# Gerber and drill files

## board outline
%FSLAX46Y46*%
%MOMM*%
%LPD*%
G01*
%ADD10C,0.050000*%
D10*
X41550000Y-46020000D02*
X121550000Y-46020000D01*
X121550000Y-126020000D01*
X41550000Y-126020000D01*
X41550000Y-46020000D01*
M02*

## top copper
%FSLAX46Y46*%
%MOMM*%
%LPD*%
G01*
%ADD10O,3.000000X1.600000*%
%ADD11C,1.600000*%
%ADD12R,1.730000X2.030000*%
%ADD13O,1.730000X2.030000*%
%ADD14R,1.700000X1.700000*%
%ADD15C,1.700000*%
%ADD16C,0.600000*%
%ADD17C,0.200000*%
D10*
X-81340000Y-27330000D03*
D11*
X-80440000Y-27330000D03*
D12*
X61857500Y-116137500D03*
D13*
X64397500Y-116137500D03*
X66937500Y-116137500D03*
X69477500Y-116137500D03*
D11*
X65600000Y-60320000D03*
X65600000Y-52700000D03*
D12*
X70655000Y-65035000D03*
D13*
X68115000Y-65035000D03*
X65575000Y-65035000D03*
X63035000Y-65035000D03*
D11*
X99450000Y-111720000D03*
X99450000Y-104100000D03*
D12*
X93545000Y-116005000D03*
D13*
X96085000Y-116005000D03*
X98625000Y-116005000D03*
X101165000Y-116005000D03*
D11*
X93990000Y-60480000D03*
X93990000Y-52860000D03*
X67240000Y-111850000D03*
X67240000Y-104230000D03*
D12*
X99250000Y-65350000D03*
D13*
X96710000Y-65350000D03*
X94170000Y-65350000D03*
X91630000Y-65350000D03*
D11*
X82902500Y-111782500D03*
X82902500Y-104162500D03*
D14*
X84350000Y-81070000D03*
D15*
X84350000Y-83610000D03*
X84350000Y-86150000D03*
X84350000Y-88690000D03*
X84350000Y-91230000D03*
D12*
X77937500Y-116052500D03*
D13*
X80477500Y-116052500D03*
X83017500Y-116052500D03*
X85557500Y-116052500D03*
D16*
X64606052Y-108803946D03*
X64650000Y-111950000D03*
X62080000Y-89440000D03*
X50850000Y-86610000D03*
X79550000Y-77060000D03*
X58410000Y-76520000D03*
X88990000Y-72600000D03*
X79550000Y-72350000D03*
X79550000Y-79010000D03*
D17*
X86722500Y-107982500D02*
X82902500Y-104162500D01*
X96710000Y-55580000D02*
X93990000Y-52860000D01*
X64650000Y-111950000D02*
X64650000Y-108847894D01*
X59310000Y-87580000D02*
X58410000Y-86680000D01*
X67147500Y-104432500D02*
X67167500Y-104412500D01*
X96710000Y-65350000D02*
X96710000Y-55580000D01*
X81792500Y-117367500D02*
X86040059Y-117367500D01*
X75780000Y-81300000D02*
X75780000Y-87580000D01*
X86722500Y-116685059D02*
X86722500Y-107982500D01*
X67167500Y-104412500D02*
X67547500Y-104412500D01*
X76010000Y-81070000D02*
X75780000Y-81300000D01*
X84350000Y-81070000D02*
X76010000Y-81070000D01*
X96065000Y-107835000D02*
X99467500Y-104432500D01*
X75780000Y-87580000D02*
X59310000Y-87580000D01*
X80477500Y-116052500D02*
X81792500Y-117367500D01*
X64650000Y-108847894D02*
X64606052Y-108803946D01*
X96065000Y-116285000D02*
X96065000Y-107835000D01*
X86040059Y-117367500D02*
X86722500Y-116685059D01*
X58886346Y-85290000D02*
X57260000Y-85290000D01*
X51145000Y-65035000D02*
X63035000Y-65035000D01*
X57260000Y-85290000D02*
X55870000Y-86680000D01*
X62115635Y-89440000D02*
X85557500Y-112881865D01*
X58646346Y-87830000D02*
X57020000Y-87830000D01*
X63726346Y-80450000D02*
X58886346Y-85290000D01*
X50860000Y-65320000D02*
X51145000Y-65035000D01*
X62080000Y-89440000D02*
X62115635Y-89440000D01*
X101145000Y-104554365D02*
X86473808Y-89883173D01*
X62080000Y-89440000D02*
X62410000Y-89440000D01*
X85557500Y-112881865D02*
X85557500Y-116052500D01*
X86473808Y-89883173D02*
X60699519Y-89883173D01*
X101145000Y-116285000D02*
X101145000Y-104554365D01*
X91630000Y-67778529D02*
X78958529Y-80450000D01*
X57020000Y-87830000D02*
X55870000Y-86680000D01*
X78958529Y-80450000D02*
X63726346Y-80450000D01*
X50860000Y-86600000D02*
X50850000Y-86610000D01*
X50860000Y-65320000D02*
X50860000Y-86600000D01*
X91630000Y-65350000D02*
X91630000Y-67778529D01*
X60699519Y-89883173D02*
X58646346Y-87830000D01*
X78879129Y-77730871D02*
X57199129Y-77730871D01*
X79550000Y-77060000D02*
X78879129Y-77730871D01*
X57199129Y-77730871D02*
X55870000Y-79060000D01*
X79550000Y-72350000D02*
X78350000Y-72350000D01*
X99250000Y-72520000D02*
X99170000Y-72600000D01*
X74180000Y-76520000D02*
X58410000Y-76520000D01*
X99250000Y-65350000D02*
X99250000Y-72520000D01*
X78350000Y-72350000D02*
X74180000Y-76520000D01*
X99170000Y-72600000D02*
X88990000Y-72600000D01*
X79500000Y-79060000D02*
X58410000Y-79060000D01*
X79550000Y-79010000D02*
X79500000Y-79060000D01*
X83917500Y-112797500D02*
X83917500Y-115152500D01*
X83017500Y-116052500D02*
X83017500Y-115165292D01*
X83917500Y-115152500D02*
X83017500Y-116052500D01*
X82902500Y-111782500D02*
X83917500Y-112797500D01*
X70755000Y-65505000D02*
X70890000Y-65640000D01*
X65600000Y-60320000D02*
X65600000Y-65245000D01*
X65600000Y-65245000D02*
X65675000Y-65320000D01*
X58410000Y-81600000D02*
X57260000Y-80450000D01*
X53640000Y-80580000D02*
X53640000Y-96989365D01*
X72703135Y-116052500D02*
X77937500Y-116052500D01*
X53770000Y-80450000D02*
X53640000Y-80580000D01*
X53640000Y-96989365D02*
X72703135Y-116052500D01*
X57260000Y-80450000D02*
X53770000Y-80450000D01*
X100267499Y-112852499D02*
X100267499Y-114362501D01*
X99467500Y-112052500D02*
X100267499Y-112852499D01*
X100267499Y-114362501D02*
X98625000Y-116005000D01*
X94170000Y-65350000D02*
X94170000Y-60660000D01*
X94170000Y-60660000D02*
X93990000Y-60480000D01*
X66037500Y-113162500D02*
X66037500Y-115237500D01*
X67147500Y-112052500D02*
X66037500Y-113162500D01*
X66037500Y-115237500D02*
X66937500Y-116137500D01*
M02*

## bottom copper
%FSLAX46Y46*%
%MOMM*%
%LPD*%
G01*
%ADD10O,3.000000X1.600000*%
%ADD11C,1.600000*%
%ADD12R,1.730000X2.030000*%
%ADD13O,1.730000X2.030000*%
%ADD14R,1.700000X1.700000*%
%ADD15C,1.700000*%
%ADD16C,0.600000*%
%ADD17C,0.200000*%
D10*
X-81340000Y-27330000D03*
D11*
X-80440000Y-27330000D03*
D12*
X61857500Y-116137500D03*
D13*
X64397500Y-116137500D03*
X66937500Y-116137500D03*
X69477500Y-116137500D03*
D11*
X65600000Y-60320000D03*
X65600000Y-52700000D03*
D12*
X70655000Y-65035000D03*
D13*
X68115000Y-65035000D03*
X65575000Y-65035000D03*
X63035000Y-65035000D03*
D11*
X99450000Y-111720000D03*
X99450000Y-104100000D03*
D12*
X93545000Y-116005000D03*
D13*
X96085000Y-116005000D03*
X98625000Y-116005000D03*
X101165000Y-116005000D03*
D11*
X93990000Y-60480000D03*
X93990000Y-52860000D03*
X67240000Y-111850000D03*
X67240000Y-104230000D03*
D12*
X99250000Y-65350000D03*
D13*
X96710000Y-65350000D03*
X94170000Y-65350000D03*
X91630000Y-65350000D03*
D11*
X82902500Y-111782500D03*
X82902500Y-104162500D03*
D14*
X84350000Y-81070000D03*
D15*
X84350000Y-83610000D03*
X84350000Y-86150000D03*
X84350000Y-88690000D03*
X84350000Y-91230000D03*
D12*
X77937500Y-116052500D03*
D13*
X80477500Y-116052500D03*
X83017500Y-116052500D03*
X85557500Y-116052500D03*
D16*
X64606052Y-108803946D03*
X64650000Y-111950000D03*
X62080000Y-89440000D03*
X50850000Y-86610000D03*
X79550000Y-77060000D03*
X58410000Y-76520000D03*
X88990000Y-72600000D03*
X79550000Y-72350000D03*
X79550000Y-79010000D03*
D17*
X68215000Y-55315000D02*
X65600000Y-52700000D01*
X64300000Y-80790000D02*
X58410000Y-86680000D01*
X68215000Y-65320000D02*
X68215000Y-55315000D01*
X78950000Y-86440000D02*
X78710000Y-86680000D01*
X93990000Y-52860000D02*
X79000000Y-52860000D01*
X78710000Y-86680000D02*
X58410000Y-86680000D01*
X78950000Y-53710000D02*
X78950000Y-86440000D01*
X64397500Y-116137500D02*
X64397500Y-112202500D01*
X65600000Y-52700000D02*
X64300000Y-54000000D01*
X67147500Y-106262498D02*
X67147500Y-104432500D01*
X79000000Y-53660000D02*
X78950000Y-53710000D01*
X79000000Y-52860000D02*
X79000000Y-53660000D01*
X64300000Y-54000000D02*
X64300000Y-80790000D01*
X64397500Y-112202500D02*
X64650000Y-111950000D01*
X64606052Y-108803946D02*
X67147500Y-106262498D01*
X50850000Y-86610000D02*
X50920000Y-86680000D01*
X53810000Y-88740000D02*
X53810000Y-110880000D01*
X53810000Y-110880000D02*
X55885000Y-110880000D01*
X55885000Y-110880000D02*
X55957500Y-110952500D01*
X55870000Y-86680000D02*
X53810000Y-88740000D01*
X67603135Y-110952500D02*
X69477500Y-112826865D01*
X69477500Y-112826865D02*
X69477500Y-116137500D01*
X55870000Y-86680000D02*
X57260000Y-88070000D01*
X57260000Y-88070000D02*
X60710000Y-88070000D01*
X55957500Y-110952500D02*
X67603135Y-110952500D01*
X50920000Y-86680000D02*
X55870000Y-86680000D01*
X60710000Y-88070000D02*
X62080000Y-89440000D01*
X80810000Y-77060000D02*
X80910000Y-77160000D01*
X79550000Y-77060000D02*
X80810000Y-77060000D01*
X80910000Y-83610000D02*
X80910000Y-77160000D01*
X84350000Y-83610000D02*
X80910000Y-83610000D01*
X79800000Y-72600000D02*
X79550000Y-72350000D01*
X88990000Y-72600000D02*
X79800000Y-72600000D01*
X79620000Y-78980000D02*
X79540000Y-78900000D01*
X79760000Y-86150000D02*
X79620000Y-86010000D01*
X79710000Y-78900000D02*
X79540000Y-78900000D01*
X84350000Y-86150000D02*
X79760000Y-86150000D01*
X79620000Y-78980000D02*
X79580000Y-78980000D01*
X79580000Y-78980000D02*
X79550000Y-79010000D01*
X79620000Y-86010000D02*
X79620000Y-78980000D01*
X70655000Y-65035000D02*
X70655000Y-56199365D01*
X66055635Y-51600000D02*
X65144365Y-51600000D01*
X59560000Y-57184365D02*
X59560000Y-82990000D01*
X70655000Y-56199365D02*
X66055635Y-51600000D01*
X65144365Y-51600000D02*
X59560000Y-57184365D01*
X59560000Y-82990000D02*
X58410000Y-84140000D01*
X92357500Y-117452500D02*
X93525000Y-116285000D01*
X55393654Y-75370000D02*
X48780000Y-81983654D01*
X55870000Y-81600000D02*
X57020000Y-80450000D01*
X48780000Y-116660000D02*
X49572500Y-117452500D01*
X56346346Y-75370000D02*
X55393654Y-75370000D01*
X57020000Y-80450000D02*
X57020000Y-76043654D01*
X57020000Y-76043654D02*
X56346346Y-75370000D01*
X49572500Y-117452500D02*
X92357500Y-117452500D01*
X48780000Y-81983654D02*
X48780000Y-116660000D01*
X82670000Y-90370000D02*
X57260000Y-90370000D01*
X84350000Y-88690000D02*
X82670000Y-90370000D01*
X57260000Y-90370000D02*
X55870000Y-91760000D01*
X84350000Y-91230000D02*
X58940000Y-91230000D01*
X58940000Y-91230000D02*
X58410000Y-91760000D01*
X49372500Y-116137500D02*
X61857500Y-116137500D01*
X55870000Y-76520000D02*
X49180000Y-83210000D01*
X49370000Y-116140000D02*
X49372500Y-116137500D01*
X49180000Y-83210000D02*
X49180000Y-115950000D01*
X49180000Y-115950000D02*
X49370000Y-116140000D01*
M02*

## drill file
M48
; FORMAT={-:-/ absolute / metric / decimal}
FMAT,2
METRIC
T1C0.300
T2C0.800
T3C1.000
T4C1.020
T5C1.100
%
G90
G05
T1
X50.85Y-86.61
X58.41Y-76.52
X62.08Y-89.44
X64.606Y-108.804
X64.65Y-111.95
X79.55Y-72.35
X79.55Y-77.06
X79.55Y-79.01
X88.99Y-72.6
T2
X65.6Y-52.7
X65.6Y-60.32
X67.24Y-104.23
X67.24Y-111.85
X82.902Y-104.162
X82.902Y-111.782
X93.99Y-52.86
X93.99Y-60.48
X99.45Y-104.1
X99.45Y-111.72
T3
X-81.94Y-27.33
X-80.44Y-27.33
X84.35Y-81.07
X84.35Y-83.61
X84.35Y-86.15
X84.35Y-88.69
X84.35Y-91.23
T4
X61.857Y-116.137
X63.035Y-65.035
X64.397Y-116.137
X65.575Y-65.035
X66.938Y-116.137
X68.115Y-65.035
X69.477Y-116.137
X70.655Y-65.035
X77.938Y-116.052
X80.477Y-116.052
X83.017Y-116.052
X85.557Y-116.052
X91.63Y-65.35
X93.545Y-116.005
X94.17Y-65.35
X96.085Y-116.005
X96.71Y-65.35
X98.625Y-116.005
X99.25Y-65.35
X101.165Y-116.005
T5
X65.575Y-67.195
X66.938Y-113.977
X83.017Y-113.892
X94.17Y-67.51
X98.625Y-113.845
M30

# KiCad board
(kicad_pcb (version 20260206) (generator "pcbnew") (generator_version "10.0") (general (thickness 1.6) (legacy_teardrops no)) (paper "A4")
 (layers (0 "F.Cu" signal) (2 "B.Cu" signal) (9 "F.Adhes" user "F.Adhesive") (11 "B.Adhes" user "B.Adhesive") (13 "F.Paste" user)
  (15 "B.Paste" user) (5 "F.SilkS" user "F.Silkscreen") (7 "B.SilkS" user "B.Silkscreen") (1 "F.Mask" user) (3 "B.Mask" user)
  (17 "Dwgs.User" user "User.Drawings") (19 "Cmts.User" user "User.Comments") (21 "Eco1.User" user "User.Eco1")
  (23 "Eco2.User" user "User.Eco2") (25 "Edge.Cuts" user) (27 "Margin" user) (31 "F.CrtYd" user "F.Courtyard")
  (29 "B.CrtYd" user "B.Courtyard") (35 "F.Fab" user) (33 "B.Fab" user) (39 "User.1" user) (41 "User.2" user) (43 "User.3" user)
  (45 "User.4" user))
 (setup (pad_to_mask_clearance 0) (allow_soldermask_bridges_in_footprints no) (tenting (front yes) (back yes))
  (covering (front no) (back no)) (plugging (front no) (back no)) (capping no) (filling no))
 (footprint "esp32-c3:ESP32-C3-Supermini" (layer "F.Cu") (at -89.44 37.33)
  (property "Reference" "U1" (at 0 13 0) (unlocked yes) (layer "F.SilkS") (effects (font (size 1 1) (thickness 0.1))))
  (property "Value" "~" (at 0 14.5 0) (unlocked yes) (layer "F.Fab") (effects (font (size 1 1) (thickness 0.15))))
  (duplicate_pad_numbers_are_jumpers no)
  (pad "1" thru_hole oval (at 7.5 -10) (size 3 1.6) (drill 1 (offset 0.6 0)) (layers "*.Cu" "*.Mask") (remove_unused_layers no)
   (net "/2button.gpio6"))
  (pad "1" thru_hole circle (at 9 -10) (size 1.6 1.6) (drill 1) (layers "*.Cu" "*.Mask") (remove_unused_layers no) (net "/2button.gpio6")))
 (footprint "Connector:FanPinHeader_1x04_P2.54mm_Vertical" (layer "F.Cu") (at 61.8575 116.1375)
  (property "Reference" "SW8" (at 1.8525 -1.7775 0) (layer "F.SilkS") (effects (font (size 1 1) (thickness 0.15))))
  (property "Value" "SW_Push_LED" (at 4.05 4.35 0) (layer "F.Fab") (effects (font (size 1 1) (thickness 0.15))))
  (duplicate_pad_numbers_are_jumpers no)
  (pad "" np_thru_hole circle (at 5.08 -2.16 90) (size 1.1 1.1) (drill 1.1) (layers "*.Cu" "*.Mask"))
  (pad "1" thru_hole rect (at 0 0 90) (size 2.03 1.73) (drill 1.02) (layers "*.Cu" "*.Mask") (remove_unused_layers no)
   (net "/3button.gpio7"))
  (pad "2" thru_hole oval (at 2.54 0 90) (size 2.03 1.73) (drill 1.02) (layers "*.Cu" "*.Mask") (remove_unused_layers no) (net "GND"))
  (pad "3" thru_hole oval (at 5.08 0 90) (size 2.03 1.73) (drill 1.02) (layers "*.Cu" "*.Mask") (remove_unused_layers no)
   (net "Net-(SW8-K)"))
  (pad "4" thru_hole oval (at 7.62 0 90) (size 2.03 1.73) (drill 1.02) (layers "*.Cu" "*.Mask") (remove_unused_layers no) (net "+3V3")))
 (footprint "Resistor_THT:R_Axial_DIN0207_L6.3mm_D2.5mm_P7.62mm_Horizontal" (layer "F.Cu") (at 65.6 60.32 90)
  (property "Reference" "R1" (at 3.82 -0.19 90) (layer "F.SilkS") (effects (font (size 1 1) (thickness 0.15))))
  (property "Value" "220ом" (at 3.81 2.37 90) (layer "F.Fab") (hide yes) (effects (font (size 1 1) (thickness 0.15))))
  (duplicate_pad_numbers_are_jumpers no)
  (pad "1" thru_hole circle (at 0 0 90) (size 1.6 1.6) (drill 0.8) (layers "*.Cu" "*.Mask") (remove_unused_layers no) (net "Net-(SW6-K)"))
  (pad "2" thru_hole circle (at 7.62 0 90) (size 1.6 1.6) (drill 0.8) (layers "*.Cu" "*.Mask") (remove_unused_layers no) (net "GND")))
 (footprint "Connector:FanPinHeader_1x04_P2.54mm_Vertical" (layer "F.Cu") (at 70.655 65.035 180)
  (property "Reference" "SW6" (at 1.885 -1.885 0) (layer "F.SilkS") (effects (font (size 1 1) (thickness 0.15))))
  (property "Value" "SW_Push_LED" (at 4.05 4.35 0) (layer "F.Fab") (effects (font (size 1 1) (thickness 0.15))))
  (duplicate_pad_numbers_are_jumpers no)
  (pad "" np_thru_hole circle (at 5.08 -2.16 270) (size 1.1 1.1) (drill 1.1) (layers "*.Cu" "*.Mask"))
  (pad "1" thru_hole rect (at 0 0 270) (size 2.03 1.73) (drill 1.02) (layers "*.Cu" "*.Mask") (remove_unused_layers no)
   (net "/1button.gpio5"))
  (pad "2" thru_hole oval (at 2.54 0 270) (size 2.03 1.73) (drill 1.02) (layers "*.Cu" "*.Mask") (remove_unused_layers no) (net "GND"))
  (pad "3" thru_hole oval (at 5.08 0 270) (size 2.03 1.73) (drill 1.02) (layers "*.Cu" "*.Mask") (remove_unused_layers no)
   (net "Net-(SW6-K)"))
  (pad "4" thru_hole oval (at 7.62 0 270) (size 2.03 1.73) (drill 1.02) (layers "*.Cu" "*.Mask") (remove_unused_layers no) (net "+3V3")))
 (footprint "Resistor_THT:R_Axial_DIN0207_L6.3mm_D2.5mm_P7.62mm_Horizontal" (layer "F.Cu") (at 99.45 111.72 90)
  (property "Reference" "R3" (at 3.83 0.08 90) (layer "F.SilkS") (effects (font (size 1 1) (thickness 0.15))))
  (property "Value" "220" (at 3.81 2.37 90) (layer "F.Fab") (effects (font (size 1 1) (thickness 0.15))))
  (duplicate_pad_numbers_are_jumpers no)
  (pad "1" thru_hole circle (at 0 0 90) (size 1.6 1.6) (drill 0.8) (layers "*.Cu" "*.Mask") (remove_unused_layers no) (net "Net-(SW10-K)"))
  (pad "2" thru_hole circle (at 7.62 0 90) (size 1.6 1.6) (drill 0.8) (layers "*.Cu" "*.Mask") (remove_unused_layers no) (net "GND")))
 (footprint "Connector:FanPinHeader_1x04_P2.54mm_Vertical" (layer "F.Cu") (at 93.545 116.005)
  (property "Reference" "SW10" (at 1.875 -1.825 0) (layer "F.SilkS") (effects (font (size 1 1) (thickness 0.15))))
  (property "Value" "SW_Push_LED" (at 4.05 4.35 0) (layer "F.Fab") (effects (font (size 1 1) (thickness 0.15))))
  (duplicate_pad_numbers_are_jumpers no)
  (pad "" np_thru_hole circle (at 5.08 -2.16 90) (size 1.1 1.1) (drill 1.1) (layers "*.Cu" "*.Mask"))
  (pad "1" thru_hole rect (at 0 0 90) (size 2.03 1.73) (drill 1.02) (layers "*.Cu" "*.Mask") (remove_unused_layers no)
   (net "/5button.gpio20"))
  (pad "2" thru_hole oval (at 2.54 0 90) (size 2.03 1.73) (drill 1.02) (layers "*.Cu" "*.Mask") (remove_unused_layers no) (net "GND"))
  (pad "3" thru_hole oval (at 5.08 0 90) (size 2.03 1.73) (drill 1.02) (layers "*.Cu" "*.Mask") (remove_unused_layers no)
   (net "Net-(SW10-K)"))
  (pad "4" thru_hole oval (at 7.62 0 90) (size 2.03 1.73) (drill 1.02) (layers "*.Cu" "*.Mask") (remove_unused_layers no) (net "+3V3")))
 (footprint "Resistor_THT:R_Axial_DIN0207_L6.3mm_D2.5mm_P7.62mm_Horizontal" (layer "F.Cu") (at 93.99 60.48 90)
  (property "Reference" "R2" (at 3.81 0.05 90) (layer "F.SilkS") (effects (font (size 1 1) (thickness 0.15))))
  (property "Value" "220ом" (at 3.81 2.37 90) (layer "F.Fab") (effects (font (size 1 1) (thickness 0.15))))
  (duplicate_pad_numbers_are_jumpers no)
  (pad "1" thru_hole circle (at 0 0 90) (size 1.6 1.6) (drill 0.8) (layers "*.Cu" "*.Mask") (remove_unused_layers no) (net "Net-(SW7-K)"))
  (pad "2" thru_hole circle (at 7.62 0 90) (size 1.6 1.6) (drill 0.8) (layers "*.Cu" "*.Mask") (remove_unused_layers no) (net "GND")))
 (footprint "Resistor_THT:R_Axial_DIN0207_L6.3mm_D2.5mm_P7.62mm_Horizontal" (layer "F.Cu") (at 67.24 111.85 90)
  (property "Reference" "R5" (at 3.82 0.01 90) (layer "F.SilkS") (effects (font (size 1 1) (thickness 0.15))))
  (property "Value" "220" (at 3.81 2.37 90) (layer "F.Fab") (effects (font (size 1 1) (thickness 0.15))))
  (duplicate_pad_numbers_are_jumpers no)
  (pad "1" thru_hole circle (at 0 0 90) (size 1.6 1.6) (drill 0.8) (layers "*.Cu" "*.Mask") (remove_unused_layers no) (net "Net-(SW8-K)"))
  (pad "2" thru_hole circle (at 7.62 0 90) (size 1.6 1.6) (drill 0.8) (layers "*.Cu" "*.Mask") (remove_unused_layers no) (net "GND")))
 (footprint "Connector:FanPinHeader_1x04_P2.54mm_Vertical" (layer "F.Cu") (at 99.25 65.35 180)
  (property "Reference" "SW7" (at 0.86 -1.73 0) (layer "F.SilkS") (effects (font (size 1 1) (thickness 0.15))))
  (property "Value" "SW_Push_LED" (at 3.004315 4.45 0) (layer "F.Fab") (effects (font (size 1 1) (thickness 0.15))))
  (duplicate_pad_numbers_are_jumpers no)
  (pad "" np_thru_hole circle (at 5.08 -2.16 270) (size 1.1 1.1) (drill 1.1) (layers "*.Cu" "*.Mask"))
  (pad "1" thru_hole rect (at 0 0 270) (size 2.03 1.73) (drill 1.02) (layers "*.Cu" "*.Mask") (remove_unused_layers no)
   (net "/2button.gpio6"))
  (pad "2" thru_hole oval (at 2.54 0 270) (size 2.03 1.73) (drill 1.02) (layers "*.Cu" "*.Mask") (remove_unused_layers no) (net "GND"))
  (pad "3" thru_hole oval (at 5.08 0 270) (size 2.03 1.73) (drill 1.02) (layers "*.Cu" "*.Mask") (remove_unused_layers no)
   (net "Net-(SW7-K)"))
  (pad "4" thru_hole oval (at 7.62 0 270) (size 2.03 1.73) (drill 1.02) (layers "*.Cu" "*.Mask") (remove_unused_layers no) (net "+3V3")))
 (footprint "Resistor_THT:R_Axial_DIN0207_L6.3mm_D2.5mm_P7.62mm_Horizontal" (layer "F.Cu") (at 82.9025 111.7825 90)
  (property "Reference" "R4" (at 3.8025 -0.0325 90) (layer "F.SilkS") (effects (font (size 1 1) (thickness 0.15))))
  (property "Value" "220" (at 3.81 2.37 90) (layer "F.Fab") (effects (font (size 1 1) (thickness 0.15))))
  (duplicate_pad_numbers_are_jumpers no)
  (pad "1" thru_hole circle (at 0 0 90) (size 1.6 1.6) (drill 0.8) (layers "*.Cu" "*.Mask") (remove_unused_layers no) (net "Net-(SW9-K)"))
  (pad "2" thru_hole circle (at 7.62 0 90) (size 1.6 1.6) (drill 0.8) (layers "*.Cu" "*.Mask") (remove_unused_layers no) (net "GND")))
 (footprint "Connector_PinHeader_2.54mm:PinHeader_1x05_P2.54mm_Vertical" (layer "F.Cu") (at 84.35 81.07)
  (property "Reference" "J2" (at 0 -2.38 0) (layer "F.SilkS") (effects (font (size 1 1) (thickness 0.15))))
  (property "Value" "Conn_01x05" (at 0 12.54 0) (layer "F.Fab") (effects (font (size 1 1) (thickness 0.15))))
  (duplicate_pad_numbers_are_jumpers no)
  (pad "1" thru_hole rect (at 0 0) (size 1.7 1.7) (drill 1) (layers "*.Cu" "*.Mask") (remove_unused_layers no) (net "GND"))
  (pad "2" thru_hole circle (at 0 2.54) (size 1.7 1.7) (drill 1) (layers "*.Cu" "*.Mask") (remove_unused_layers no) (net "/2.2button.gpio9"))
  (pad "3" thru_hole circle (at 0 5.08) (size 1.7 1.7) (drill 1) (layers "*.Cu" "*.Mask") (remove_unused_layers no) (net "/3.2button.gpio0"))
  (pad "4" thru_hole circle (at 0 7.62) (size 1.7 1.7) (drill 1) (layers "*.Cu" "*.Mask") (remove_unused_layers no) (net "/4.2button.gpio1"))
  (pad "5" thru_hole circle (at 0 10.16) (size 1.7 1.7) (drill 1) (layers "*.Cu" "*.Mask") (remove_unused_layers no)
   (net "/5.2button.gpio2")))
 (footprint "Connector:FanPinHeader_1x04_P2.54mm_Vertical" (layer "F.Cu") (at 77.9375 116.0525)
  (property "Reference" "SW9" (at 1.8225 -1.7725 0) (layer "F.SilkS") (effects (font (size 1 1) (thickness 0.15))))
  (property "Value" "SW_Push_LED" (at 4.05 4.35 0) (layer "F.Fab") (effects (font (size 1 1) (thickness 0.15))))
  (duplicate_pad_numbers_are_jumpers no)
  (pad "" np_thru_hole circle (at 5.08 -2.16 90) (size 1.1 1.1) (drill 1.1) (layers "*.Cu" "*.Mask"))
  (pad "1" thru_hole rect (at 0 0 90) (size 2.03 1.73) (drill 1.02) (layers "*.Cu" "*.Mask") (remove_unused_layers no)
   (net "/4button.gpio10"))
  (pad "2" thru_hole oval (at 2.54 0 90) (size 2.03 1.73) (drill 1.02) (layers "*.Cu" "*.Mask") (remove_unused_layers no) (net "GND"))
  (pad "3" thru_hole oval (at 5.08 0 90) (size 2.03 1.73) (drill 1.02) (layers "*.Cu" "*.Mask") (remove_unused_layers no)
   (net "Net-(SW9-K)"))
  (pad "4" thru_hole oval (at 7.62 0 90) (size 2.03 1.73) (drill 1.02) (layers "*.Cu" "*.Mask") (remove_unused_layers no) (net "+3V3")))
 (gr_rect (start 41.55 46.02) (end 121.55 126.02) (stroke (width 0.05) (type default)) (fill no) (layer "Edge.Cuts"))
 (segment (start 86.7225 107.9825) (end 82.9025 104.1625) (width 0.2) (layer "F.Cu") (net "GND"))
 (segment (start 96.71 55.58) (end 93.99 52.86) (width 0.2) (layer "F.Cu") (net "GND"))
 (segment (start 64.65 111.95) (end 64.65 108.847894) (width 0.2) (layer "F.Cu") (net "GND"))
 (segment (start 59.31 87.58) (end 58.41 86.68) (width 0.2) (layer "F.Cu") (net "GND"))
 (segment (start 67.1475 104.4325) (end 67.1675 104.4125) (width 0.2) (layer "F.Cu") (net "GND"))
 (segment (start 96.71 65.35) (end 96.71 55.58) (width 0.2) (layer "F.Cu") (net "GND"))
 (segment (start 81.7925 117.3675) (end 86.040059 117.3675) (width 0.2) (layer "F.Cu") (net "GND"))
 (segment (start 75.78 81.3) (end 75.78 87.58) (width 0.2) (layer "F.Cu") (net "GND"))
 (segment (start 86.7225 116.685059) (end 86.7225 107.9825) (width 0.2) (layer "F.Cu") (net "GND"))
 (segment (start 67.1675 104.4125) (end 67.5475 104.4125) (width 0.2) (layer "F.Cu") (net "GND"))
 (segment (start 76.01 81.07) (end 75.78 81.3) (width 0.2) (layer "F.Cu") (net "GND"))
 (segment (start 84.35 81.07) (end 76.01 81.07) (width 0.2) (layer "F.Cu") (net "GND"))
 (segment (start 96.065 107.835) (end 99.4675 104.4325) (width 0.2) (layer "F.Cu") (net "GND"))
 (segment (start 75.78 87.58) (end 59.31 87.58) (width 0.2) (layer "F.Cu") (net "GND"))
 (segment (start 80.4775 116.0525) (end 81.7925 117.3675) (width 0.2) (layer "F.Cu") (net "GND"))
 (segment (start 64.65 108.847894) (end 64.606052 108.803946) (width 0.2) (layer "F.Cu") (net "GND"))
 (segment (start 96.065 116.285) (end 96.065 107.835) (width 0.2) (layer "F.Cu") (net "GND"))
 (segment (start 86.040059 117.3675) (end 86.7225 116.685059) (width 0.2) (layer "F.Cu") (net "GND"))
 (via (at 64.606052 108.803946) (size 0.6) (drill 0.3) (layers "F.Cu" "B.Cu") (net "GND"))
 (via (at 64.65 111.95) (size 0.6) (drill 0.3) (layers "F.Cu" "B.Cu") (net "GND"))
 (segment (start 68.215 55.315) (end 65.6 52.7) (width 0.2) (layer "B.Cu") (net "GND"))
 (segment (start 64.3 80.79) (end 58.41 86.68) (width 0.2) (layer "B.Cu") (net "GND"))
 (segment (start 68.215 65.32) (end 68.215 55.315) (width 0.2) (layer "B.Cu") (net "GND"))
 (segment (start 78.95 86.44) (end 78.71 86.68) (width 0.2) (layer "B.Cu") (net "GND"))
 (segment (start 93.99 52.86) (end 79 52.86) (width 0.2) (layer "B.Cu") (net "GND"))
 (segment (start 78.71 86.68) (end 58.41 86.68) (width 0.2) (layer "B.Cu") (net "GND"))
 (segment (start 78.95 53.71) (end 78.95 86.44) (width 0.2) (layer "B.Cu") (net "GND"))
 (segment (start 64.3975 116.1375) (end 64.3975 112.2025) (width 0.2) (layer "B.Cu") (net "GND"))
 (segment (start 65.6 52.7) (end 64.3 54) (width 0.2) (layer "B.Cu") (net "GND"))
 (segment (start 67.1475 106.262498) (end 67.1475 104.4325) (width 0.2) (layer "B.Cu") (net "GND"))
 (segment (start 79 53.66) (end 78.95 53.71) (width 0.2) (layer "B.Cu") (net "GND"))
 (segment (start 79 52.86) (end 79 53.66) (width 0.2) (layer "B.Cu") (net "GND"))
 (segment (start 64.3 54) (end 64.3 80.79) (width 0.2) (layer "B.Cu") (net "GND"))
 (segment (start 64.3975 112.2025) (end 64.65 111.95) (width 0.2) (layer "B.Cu") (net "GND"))
 (segment (start 64.606052 108.803946) (end 67.1475 106.262498) (width 0.2) (layer "B.Cu") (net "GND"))
 (segment (start 58.886346 85.29) (end 57.26 85.29) (width 0.2) (layer "F.Cu") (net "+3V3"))
 (segment (start 51.145 65.035) (end 63.035 65.035) (width 0.2) (layer "F.Cu") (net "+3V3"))
 (segment (start 57.26 85.29) (end 55.87 86.68) (width 0.2) (layer "F.Cu") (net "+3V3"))
 (segment (start 62.115635 89.44) (end 85.5575 112.881865) (width 0.2) (layer "F.Cu") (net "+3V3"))
 (segment (start 58.646346 87.83) (end 57.02 87.83) (width 0.2) (layer "F.Cu") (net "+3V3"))
 (segment (start 63.726346 80.45) (end 58.886346 85.29) (width 0.2) (layer "F.Cu") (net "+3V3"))
 (segment (start 50.86 65.32) (end 51.145 65.035) (width 0.2) (layer "F.Cu") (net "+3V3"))
 (segment (start 62.08 89.44) (end 62.115635 89.44) (width 0.2) (layer "F.Cu") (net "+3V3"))
 (segment (start 101.145 104.554365) (end 86.473808 89.883173) (width 0.2) (layer "F.Cu") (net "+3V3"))
 (segment (start 62.08 89.44) (end 62.41 89.44) (width 0.2) (layer "F.Cu") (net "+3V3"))
 (segment (start 85.5575 112.881865) (end 85.5575 116.0525) (width 0.2) (layer "F.Cu") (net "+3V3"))
 (segment (start 86.473808 89.883173) (end 60.699519 89.883173) (width 0.2) (layer "F.Cu") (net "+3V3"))
 (segment (start 101.145 116.285) (end 101.145 104.554365) (width 0.2) (layer "F.Cu") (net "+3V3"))
 (segment (start 91.63 67.778529) (end 78.958529 80.45) (width 0.2) (layer "F.Cu") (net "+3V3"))
 (segment (start 57.02 87.83) (end 55.87 86.68) (width 0.2) (layer "F.Cu") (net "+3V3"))
 (segment (start 78.958529 80.45) (end 63.726346 80.45) (width 0.2) (layer "F.Cu") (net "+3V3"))
 (segment (start 50.86 86.6) (end 50.85 86.61) (width 0.2) (layer "F.Cu") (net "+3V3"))
 (segment (start 50.86 65.32) (end 50.86 86.6) (width 0.2) (layer "F.Cu") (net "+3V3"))
 (segment (start 91.63 65.35) (end 91.63 67.778529) (width 0.2) (layer "F.Cu") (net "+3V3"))
 (segment (start 60.699519 89.883173) (end 58.646346 87.83) (width 0.2) (layer "F.Cu") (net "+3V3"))
 (via (at 62.08 89.44) (size 0.6) (drill 0.3) (layers "F.Cu" "B.Cu") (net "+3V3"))
 (via (at 50.85 86.61) (size 0.6) (drill 0.3) (layers "F.Cu" "B.Cu") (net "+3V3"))
 (segment (start 50.85 86.61) (end 50.92 86.68) (width 0.2) (layer "B.Cu") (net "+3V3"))
 (segment (start 53.81 88.74) (end 53.81 110.88) (width 0.2) (layer "B.Cu") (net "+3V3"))
 (segment (start 53.81 110.88) (end 55.885 110.88) (width 0.2) (layer "B.Cu") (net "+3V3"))
 (segment (start 55.885 110.88) (end 55.9575 110.9525) (width 0.2) (layer "B.Cu") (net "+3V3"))
 (segment (start 55.87 86.68) (end 53.81 88.74) (width 0.2) (layer "B.Cu") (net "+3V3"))
 (segment (start 67.603135 110.9525) (end 69.4775 112.826865) (width 0.2) (layer "B.Cu") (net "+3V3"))
 (segment (start 69.4775 112.826865) (end 69.4775 116.1375) (width 0.2) (layer "B.Cu") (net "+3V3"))
 (segment (start 55.87 86.68) (end 57.26 88.07) (width 0.2) (layer "B.Cu") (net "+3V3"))
 (segment (start 57.26 88.07) (end 60.71 88.07) (width 0.2) (layer "B.Cu") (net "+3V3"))
 (segment (start 55.9575 110.9525) (end 67.603135 110.9525) (width 0.2) (layer "B.Cu") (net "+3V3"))
 (segment (start 50.92 86.68) (end 55.87 86.68) (width 0.2) (layer "B.Cu") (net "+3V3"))
 (segment (start 60.71 88.07) (end 62.08 89.44) (width 0.2) (layer "B.Cu") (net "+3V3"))
 (segment (start 78.879129 77.730871) (end 57.199129 77.730871) (width 0.2) (layer "F.Cu") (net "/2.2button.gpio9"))
 (segment (start 79.55 77.06) (end 78.879129 77.730871) (width 0.2) (layer "F.Cu") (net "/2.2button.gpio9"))
 (segment (start 57.199129 77.730871) (end 55.87 79.06) (width 0.2) (layer "F.Cu") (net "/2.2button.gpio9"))
 (via (at 79.55 77.06) (size 0.6) (drill 0.3) (layers "F.Cu" "B.Cu") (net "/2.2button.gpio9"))
 (segment (start 80.81 77.06) (end 80.91 77.16) (width 0.2) (layer "B.Cu") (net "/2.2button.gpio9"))
 (segment (start 79.55 77.06) (end 80.81 77.06) (width 0.2) (layer "B.Cu") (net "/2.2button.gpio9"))
 (segment (start 80.91 83.61) (end 80.91 77.16) (width 0.2) (layer "B.Cu") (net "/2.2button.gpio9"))
 (segment (start 84.35 83.61) (end 80.91 83.61) (width 0.2) (layer "B.Cu") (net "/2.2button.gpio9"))
 (segment (start 79.55 72.35) (end 78.35 72.35) (width 0.2) (layer "F.Cu") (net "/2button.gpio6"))
 (segment (start 99.25 72.52) (end 99.17 72.6) (width 0.2) (layer "F.Cu") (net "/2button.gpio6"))
 (segment (start 74.18 76.52) (end 58.41 76.52) (width 0.2) (layer "F.Cu") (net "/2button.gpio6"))
 (segment (start 99.25 65.35) (end 99.25 72.52) (width 0.2) (layer "F.Cu") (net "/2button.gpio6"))
 (segment (start 78.35 72.35) (end 74.18 76.52) (width 0.2) (layer "F.Cu") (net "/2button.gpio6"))
 (segment (start 99.17 72.6) (end 88.99 72.6) (width 0.2) (layer "F.Cu") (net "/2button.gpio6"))
 (via (at 58.41 76.52) (size 0.6) (drill 0.3) (layers "F.Cu" "B.Cu") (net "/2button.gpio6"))
 (via (at 88.99 72.6) (size 0.6) (drill 0.3) (layers "F.Cu" "B.Cu") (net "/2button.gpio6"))
 (via (at 79.55 72.35) (size 0.6) (drill 0.3) (layers "F.Cu" "B.Cu") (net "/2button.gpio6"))
 (segment (start 79.8 72.6) (end 79.55 72.35) (width 0.2) (layer "B.Cu") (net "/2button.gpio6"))
 (segment (start 88.99 72.6) (end 79.8 72.6) (width 0.2) (layer "B.Cu") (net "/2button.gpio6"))
 (segment (start 79.5 79.06) (end 58.41 79.06) (width 0.2) (layer "F.Cu") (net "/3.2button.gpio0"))
 (segment (start 79.55 79.01) (end 79.5 79.06) (width 0.2) (layer "F.Cu") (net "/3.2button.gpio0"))
 (via (at 79.55 79.01) (size 0.6) (drill 0.3) (layers "F.Cu" "B.Cu") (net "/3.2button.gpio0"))
 (segment (start 79.62 78.98) (end 79.54 78.9) (width 0.2) (layer "B.Cu") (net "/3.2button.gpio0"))
 (segment (start 79.76 86.15) (end 79.62 86.01) (width 0.2) (layer "B.Cu") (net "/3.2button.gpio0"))
 (segment (start 79.71 78.9) (end 79.54 78.9) (width 0.2) (layer "B.Cu") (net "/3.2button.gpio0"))
 (segment (start 84.35 86.15) (end 79.76 86.15) (width 0.2) (layer "B.Cu") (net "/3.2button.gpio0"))
 (segment (start 79.62 78.98) (end 79.58 78.98) (width 0.2) (layer "B.Cu") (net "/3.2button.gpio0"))
 (segment (start 79.58 78.98) (end 79.55 79.01) (width 0.2) (layer "B.Cu") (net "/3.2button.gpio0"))
 (segment (start 79.62 86.01) (end 79.62 78.98) (width 0.2) (layer "B.Cu") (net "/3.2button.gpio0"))
 (segment (start 83.9175 112.7975) (end 83.9175 115.1525) (width 0.2) (layer "F.Cu") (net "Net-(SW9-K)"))
 (segment (start 83.0175 116.0525) (end 83.0175 115.165292) (width 0.2) (layer "F.Cu") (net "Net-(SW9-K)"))
 (segment (start 83.9175 115.1525) (end 83.0175 116.0525) (width 0.2) (layer "F.Cu") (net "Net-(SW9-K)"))
 (segment (start 82.9025 111.7825) (end 83.9175 112.7975) (width 0.2) (layer "F.Cu") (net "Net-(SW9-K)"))
 (segment (start 70.755 65.505) (end 70.89 65.64) (width 0.2) (layer "F.Cu") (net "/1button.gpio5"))
 (segment (start 70.655 65.035) (end 70.655 56.199365) (width 0.2) (layer "B.Cu") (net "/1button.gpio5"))
 (segment (start 66.055635 51.6) (end 65.144365 51.6) (width 0.2) (layer "B.Cu") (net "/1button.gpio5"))
 (segment (start 59.56 57.184365) (end 59.56 82.99) (width 0.2) (layer "B.Cu") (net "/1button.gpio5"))
 (segment (start 70.655 56.199365) (end 66.055635 51.6) (width 0.2) (layer "B.Cu") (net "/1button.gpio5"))
 (segment (start 65.144365 51.6) (end 59.56 57.184365) (width 0.2) (layer "B.Cu") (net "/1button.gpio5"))
 (segment (start 59.56 82.99) (end 58.41 84.14) (width 0.2) (layer "B.Cu") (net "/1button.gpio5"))
 (segment (start 65.6 60.32) (end 65.6 65.245) (width 0.2) (layer "F.Cu") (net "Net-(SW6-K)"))
 (segment (start 65.6 65.245) (end 65.675 65.32) (width 0.2) (layer "F.Cu") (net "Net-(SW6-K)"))
 (segment (start 92.3575 117.4525) (end 93.525 116.285) (width 0.2) (layer "B.Cu") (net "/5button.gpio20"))
 (segment (start 55.393654 75.37) (end 48.78 81.983654) (width 0.2) (layer "B.Cu") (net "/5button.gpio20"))
 (segment (start 55.87 81.6) (end 57.02 80.45) (width 0.2) (layer "B.Cu") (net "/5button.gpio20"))
 (segment (start 48.78 116.66) (end 49.5725 117.4525) (width 0.2) (layer "B.Cu") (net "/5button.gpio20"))
 (segment (start 56.346346 75.37) (end 55.393654 75.37) (width 0.2) (layer "B.Cu") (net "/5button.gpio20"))
 (segment (start 57.02 80.45) (end 57.02 76.043654) (width 0.2) (layer "B.Cu") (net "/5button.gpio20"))
 (segment (start 57.02 76.043654) (end 56.346346 75.37) (width 0.2) (layer "B.Cu") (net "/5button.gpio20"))
 (segment (start 49.5725 117.4525) (end 92.3575 117.4525) (width 0.2) (layer "B.Cu") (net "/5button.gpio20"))
 (segment (start 48.78 81.983654) (end 48.78 116.66) (width 0.2) (layer "B.Cu") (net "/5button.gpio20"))
 (segment (start 82.67 90.37) (end 57.26 90.37) (width 0.2) (layer "B.Cu") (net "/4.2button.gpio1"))
 (segment (start 84.35 88.69) (end 82.67 90.37) (width 0.2) (layer "B.Cu") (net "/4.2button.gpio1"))
 (segment (start 57.26 90.37) (end 55.87 91.76) (width 0.2) (layer "B.Cu") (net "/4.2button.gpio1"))
 (segment (start 84.35 91.23) (end 58.94 91.23) (width 0.2) (layer "B.Cu") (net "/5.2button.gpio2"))
 (segment (start 58.94 91.23) (end 58.41 91.76) (width 0.2) (layer "B.Cu") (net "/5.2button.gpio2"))
 (segment (start 58.41 81.6) (end 57.26 80.45) (width 0.2) (layer "F.Cu") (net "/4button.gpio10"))
 (segment (start 53.64 80.58) (end 53.64 96.989365) (width 0.2) (layer "F.Cu") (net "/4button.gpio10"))
 (segment (start 72.703135 116.0525) (end 77.9375 116.0525) (width 0.2) (layer "F.Cu") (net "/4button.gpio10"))
 (segment (start 53.77 80.45) (end 53.64 80.58) (width 0.2) (layer "F.Cu") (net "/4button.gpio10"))
 (segment (start 53.64 96.989365) (end 72.703135 116.0525) (width 0.2) (layer "F.Cu") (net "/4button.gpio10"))
 (segment (start 57.26 80.45) (end 53.77 80.45) (width 0.2) (layer "F.Cu") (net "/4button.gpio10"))
 (segment (start 100.267499 112.852499) (end 100.267499 114.362501) (width 0.2) (layer "F.Cu") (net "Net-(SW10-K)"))
 (segment (start 99.4675 112.0525) (end 100.267499 112.852499) (width 0.2) (layer "F.Cu") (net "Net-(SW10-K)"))
 (segment (start 100.267499 114.362501) (end 98.625 116.005) (width 0.2) (layer "F.Cu") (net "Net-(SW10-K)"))
 (segment (start 94.17 65.35) (end 94.17 60.66) (width 0.2) (layer "F.Cu") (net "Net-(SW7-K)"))
 (segment (start 94.17 60.66) (end 93.99 60.48) (width 0.2) (layer "F.Cu") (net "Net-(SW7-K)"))
 (segment (start 49.3725 116.1375) (end 61.8575 116.1375) (width 0.2) (layer "B.Cu") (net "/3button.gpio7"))
 (segment (start 55.87 76.52) (end 49.18 83.21) (width 0.2) (layer "B.Cu") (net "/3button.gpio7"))
 (segment (start 49.37 116.14) (end 49.3725 116.1375) (width 0.2) (layer "B.Cu") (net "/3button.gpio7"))
 (segment (start 49.18 83.21) (end 49.18 115.95) (width 0.2) (layer "B.Cu") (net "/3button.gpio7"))
 (segment (start 49.18 115.95) (end 49.37 116.14) (width 0.2) (layer "B.Cu") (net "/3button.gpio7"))
 (segment (start 66.0375 113.1625) (end 66.0375 115.2375) (width 0.2) (layer "F.Cu") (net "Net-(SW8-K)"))
 (segment (start 67.1475 112.0525) (end 66.0375 113.1625) (width 0.2) (layer "F.Cu") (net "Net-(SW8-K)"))
 (segment (start 66.0375 115.2375) (end 66.9375 116.1375) (width 0.2) (layer "F.Cu") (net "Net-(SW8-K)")))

